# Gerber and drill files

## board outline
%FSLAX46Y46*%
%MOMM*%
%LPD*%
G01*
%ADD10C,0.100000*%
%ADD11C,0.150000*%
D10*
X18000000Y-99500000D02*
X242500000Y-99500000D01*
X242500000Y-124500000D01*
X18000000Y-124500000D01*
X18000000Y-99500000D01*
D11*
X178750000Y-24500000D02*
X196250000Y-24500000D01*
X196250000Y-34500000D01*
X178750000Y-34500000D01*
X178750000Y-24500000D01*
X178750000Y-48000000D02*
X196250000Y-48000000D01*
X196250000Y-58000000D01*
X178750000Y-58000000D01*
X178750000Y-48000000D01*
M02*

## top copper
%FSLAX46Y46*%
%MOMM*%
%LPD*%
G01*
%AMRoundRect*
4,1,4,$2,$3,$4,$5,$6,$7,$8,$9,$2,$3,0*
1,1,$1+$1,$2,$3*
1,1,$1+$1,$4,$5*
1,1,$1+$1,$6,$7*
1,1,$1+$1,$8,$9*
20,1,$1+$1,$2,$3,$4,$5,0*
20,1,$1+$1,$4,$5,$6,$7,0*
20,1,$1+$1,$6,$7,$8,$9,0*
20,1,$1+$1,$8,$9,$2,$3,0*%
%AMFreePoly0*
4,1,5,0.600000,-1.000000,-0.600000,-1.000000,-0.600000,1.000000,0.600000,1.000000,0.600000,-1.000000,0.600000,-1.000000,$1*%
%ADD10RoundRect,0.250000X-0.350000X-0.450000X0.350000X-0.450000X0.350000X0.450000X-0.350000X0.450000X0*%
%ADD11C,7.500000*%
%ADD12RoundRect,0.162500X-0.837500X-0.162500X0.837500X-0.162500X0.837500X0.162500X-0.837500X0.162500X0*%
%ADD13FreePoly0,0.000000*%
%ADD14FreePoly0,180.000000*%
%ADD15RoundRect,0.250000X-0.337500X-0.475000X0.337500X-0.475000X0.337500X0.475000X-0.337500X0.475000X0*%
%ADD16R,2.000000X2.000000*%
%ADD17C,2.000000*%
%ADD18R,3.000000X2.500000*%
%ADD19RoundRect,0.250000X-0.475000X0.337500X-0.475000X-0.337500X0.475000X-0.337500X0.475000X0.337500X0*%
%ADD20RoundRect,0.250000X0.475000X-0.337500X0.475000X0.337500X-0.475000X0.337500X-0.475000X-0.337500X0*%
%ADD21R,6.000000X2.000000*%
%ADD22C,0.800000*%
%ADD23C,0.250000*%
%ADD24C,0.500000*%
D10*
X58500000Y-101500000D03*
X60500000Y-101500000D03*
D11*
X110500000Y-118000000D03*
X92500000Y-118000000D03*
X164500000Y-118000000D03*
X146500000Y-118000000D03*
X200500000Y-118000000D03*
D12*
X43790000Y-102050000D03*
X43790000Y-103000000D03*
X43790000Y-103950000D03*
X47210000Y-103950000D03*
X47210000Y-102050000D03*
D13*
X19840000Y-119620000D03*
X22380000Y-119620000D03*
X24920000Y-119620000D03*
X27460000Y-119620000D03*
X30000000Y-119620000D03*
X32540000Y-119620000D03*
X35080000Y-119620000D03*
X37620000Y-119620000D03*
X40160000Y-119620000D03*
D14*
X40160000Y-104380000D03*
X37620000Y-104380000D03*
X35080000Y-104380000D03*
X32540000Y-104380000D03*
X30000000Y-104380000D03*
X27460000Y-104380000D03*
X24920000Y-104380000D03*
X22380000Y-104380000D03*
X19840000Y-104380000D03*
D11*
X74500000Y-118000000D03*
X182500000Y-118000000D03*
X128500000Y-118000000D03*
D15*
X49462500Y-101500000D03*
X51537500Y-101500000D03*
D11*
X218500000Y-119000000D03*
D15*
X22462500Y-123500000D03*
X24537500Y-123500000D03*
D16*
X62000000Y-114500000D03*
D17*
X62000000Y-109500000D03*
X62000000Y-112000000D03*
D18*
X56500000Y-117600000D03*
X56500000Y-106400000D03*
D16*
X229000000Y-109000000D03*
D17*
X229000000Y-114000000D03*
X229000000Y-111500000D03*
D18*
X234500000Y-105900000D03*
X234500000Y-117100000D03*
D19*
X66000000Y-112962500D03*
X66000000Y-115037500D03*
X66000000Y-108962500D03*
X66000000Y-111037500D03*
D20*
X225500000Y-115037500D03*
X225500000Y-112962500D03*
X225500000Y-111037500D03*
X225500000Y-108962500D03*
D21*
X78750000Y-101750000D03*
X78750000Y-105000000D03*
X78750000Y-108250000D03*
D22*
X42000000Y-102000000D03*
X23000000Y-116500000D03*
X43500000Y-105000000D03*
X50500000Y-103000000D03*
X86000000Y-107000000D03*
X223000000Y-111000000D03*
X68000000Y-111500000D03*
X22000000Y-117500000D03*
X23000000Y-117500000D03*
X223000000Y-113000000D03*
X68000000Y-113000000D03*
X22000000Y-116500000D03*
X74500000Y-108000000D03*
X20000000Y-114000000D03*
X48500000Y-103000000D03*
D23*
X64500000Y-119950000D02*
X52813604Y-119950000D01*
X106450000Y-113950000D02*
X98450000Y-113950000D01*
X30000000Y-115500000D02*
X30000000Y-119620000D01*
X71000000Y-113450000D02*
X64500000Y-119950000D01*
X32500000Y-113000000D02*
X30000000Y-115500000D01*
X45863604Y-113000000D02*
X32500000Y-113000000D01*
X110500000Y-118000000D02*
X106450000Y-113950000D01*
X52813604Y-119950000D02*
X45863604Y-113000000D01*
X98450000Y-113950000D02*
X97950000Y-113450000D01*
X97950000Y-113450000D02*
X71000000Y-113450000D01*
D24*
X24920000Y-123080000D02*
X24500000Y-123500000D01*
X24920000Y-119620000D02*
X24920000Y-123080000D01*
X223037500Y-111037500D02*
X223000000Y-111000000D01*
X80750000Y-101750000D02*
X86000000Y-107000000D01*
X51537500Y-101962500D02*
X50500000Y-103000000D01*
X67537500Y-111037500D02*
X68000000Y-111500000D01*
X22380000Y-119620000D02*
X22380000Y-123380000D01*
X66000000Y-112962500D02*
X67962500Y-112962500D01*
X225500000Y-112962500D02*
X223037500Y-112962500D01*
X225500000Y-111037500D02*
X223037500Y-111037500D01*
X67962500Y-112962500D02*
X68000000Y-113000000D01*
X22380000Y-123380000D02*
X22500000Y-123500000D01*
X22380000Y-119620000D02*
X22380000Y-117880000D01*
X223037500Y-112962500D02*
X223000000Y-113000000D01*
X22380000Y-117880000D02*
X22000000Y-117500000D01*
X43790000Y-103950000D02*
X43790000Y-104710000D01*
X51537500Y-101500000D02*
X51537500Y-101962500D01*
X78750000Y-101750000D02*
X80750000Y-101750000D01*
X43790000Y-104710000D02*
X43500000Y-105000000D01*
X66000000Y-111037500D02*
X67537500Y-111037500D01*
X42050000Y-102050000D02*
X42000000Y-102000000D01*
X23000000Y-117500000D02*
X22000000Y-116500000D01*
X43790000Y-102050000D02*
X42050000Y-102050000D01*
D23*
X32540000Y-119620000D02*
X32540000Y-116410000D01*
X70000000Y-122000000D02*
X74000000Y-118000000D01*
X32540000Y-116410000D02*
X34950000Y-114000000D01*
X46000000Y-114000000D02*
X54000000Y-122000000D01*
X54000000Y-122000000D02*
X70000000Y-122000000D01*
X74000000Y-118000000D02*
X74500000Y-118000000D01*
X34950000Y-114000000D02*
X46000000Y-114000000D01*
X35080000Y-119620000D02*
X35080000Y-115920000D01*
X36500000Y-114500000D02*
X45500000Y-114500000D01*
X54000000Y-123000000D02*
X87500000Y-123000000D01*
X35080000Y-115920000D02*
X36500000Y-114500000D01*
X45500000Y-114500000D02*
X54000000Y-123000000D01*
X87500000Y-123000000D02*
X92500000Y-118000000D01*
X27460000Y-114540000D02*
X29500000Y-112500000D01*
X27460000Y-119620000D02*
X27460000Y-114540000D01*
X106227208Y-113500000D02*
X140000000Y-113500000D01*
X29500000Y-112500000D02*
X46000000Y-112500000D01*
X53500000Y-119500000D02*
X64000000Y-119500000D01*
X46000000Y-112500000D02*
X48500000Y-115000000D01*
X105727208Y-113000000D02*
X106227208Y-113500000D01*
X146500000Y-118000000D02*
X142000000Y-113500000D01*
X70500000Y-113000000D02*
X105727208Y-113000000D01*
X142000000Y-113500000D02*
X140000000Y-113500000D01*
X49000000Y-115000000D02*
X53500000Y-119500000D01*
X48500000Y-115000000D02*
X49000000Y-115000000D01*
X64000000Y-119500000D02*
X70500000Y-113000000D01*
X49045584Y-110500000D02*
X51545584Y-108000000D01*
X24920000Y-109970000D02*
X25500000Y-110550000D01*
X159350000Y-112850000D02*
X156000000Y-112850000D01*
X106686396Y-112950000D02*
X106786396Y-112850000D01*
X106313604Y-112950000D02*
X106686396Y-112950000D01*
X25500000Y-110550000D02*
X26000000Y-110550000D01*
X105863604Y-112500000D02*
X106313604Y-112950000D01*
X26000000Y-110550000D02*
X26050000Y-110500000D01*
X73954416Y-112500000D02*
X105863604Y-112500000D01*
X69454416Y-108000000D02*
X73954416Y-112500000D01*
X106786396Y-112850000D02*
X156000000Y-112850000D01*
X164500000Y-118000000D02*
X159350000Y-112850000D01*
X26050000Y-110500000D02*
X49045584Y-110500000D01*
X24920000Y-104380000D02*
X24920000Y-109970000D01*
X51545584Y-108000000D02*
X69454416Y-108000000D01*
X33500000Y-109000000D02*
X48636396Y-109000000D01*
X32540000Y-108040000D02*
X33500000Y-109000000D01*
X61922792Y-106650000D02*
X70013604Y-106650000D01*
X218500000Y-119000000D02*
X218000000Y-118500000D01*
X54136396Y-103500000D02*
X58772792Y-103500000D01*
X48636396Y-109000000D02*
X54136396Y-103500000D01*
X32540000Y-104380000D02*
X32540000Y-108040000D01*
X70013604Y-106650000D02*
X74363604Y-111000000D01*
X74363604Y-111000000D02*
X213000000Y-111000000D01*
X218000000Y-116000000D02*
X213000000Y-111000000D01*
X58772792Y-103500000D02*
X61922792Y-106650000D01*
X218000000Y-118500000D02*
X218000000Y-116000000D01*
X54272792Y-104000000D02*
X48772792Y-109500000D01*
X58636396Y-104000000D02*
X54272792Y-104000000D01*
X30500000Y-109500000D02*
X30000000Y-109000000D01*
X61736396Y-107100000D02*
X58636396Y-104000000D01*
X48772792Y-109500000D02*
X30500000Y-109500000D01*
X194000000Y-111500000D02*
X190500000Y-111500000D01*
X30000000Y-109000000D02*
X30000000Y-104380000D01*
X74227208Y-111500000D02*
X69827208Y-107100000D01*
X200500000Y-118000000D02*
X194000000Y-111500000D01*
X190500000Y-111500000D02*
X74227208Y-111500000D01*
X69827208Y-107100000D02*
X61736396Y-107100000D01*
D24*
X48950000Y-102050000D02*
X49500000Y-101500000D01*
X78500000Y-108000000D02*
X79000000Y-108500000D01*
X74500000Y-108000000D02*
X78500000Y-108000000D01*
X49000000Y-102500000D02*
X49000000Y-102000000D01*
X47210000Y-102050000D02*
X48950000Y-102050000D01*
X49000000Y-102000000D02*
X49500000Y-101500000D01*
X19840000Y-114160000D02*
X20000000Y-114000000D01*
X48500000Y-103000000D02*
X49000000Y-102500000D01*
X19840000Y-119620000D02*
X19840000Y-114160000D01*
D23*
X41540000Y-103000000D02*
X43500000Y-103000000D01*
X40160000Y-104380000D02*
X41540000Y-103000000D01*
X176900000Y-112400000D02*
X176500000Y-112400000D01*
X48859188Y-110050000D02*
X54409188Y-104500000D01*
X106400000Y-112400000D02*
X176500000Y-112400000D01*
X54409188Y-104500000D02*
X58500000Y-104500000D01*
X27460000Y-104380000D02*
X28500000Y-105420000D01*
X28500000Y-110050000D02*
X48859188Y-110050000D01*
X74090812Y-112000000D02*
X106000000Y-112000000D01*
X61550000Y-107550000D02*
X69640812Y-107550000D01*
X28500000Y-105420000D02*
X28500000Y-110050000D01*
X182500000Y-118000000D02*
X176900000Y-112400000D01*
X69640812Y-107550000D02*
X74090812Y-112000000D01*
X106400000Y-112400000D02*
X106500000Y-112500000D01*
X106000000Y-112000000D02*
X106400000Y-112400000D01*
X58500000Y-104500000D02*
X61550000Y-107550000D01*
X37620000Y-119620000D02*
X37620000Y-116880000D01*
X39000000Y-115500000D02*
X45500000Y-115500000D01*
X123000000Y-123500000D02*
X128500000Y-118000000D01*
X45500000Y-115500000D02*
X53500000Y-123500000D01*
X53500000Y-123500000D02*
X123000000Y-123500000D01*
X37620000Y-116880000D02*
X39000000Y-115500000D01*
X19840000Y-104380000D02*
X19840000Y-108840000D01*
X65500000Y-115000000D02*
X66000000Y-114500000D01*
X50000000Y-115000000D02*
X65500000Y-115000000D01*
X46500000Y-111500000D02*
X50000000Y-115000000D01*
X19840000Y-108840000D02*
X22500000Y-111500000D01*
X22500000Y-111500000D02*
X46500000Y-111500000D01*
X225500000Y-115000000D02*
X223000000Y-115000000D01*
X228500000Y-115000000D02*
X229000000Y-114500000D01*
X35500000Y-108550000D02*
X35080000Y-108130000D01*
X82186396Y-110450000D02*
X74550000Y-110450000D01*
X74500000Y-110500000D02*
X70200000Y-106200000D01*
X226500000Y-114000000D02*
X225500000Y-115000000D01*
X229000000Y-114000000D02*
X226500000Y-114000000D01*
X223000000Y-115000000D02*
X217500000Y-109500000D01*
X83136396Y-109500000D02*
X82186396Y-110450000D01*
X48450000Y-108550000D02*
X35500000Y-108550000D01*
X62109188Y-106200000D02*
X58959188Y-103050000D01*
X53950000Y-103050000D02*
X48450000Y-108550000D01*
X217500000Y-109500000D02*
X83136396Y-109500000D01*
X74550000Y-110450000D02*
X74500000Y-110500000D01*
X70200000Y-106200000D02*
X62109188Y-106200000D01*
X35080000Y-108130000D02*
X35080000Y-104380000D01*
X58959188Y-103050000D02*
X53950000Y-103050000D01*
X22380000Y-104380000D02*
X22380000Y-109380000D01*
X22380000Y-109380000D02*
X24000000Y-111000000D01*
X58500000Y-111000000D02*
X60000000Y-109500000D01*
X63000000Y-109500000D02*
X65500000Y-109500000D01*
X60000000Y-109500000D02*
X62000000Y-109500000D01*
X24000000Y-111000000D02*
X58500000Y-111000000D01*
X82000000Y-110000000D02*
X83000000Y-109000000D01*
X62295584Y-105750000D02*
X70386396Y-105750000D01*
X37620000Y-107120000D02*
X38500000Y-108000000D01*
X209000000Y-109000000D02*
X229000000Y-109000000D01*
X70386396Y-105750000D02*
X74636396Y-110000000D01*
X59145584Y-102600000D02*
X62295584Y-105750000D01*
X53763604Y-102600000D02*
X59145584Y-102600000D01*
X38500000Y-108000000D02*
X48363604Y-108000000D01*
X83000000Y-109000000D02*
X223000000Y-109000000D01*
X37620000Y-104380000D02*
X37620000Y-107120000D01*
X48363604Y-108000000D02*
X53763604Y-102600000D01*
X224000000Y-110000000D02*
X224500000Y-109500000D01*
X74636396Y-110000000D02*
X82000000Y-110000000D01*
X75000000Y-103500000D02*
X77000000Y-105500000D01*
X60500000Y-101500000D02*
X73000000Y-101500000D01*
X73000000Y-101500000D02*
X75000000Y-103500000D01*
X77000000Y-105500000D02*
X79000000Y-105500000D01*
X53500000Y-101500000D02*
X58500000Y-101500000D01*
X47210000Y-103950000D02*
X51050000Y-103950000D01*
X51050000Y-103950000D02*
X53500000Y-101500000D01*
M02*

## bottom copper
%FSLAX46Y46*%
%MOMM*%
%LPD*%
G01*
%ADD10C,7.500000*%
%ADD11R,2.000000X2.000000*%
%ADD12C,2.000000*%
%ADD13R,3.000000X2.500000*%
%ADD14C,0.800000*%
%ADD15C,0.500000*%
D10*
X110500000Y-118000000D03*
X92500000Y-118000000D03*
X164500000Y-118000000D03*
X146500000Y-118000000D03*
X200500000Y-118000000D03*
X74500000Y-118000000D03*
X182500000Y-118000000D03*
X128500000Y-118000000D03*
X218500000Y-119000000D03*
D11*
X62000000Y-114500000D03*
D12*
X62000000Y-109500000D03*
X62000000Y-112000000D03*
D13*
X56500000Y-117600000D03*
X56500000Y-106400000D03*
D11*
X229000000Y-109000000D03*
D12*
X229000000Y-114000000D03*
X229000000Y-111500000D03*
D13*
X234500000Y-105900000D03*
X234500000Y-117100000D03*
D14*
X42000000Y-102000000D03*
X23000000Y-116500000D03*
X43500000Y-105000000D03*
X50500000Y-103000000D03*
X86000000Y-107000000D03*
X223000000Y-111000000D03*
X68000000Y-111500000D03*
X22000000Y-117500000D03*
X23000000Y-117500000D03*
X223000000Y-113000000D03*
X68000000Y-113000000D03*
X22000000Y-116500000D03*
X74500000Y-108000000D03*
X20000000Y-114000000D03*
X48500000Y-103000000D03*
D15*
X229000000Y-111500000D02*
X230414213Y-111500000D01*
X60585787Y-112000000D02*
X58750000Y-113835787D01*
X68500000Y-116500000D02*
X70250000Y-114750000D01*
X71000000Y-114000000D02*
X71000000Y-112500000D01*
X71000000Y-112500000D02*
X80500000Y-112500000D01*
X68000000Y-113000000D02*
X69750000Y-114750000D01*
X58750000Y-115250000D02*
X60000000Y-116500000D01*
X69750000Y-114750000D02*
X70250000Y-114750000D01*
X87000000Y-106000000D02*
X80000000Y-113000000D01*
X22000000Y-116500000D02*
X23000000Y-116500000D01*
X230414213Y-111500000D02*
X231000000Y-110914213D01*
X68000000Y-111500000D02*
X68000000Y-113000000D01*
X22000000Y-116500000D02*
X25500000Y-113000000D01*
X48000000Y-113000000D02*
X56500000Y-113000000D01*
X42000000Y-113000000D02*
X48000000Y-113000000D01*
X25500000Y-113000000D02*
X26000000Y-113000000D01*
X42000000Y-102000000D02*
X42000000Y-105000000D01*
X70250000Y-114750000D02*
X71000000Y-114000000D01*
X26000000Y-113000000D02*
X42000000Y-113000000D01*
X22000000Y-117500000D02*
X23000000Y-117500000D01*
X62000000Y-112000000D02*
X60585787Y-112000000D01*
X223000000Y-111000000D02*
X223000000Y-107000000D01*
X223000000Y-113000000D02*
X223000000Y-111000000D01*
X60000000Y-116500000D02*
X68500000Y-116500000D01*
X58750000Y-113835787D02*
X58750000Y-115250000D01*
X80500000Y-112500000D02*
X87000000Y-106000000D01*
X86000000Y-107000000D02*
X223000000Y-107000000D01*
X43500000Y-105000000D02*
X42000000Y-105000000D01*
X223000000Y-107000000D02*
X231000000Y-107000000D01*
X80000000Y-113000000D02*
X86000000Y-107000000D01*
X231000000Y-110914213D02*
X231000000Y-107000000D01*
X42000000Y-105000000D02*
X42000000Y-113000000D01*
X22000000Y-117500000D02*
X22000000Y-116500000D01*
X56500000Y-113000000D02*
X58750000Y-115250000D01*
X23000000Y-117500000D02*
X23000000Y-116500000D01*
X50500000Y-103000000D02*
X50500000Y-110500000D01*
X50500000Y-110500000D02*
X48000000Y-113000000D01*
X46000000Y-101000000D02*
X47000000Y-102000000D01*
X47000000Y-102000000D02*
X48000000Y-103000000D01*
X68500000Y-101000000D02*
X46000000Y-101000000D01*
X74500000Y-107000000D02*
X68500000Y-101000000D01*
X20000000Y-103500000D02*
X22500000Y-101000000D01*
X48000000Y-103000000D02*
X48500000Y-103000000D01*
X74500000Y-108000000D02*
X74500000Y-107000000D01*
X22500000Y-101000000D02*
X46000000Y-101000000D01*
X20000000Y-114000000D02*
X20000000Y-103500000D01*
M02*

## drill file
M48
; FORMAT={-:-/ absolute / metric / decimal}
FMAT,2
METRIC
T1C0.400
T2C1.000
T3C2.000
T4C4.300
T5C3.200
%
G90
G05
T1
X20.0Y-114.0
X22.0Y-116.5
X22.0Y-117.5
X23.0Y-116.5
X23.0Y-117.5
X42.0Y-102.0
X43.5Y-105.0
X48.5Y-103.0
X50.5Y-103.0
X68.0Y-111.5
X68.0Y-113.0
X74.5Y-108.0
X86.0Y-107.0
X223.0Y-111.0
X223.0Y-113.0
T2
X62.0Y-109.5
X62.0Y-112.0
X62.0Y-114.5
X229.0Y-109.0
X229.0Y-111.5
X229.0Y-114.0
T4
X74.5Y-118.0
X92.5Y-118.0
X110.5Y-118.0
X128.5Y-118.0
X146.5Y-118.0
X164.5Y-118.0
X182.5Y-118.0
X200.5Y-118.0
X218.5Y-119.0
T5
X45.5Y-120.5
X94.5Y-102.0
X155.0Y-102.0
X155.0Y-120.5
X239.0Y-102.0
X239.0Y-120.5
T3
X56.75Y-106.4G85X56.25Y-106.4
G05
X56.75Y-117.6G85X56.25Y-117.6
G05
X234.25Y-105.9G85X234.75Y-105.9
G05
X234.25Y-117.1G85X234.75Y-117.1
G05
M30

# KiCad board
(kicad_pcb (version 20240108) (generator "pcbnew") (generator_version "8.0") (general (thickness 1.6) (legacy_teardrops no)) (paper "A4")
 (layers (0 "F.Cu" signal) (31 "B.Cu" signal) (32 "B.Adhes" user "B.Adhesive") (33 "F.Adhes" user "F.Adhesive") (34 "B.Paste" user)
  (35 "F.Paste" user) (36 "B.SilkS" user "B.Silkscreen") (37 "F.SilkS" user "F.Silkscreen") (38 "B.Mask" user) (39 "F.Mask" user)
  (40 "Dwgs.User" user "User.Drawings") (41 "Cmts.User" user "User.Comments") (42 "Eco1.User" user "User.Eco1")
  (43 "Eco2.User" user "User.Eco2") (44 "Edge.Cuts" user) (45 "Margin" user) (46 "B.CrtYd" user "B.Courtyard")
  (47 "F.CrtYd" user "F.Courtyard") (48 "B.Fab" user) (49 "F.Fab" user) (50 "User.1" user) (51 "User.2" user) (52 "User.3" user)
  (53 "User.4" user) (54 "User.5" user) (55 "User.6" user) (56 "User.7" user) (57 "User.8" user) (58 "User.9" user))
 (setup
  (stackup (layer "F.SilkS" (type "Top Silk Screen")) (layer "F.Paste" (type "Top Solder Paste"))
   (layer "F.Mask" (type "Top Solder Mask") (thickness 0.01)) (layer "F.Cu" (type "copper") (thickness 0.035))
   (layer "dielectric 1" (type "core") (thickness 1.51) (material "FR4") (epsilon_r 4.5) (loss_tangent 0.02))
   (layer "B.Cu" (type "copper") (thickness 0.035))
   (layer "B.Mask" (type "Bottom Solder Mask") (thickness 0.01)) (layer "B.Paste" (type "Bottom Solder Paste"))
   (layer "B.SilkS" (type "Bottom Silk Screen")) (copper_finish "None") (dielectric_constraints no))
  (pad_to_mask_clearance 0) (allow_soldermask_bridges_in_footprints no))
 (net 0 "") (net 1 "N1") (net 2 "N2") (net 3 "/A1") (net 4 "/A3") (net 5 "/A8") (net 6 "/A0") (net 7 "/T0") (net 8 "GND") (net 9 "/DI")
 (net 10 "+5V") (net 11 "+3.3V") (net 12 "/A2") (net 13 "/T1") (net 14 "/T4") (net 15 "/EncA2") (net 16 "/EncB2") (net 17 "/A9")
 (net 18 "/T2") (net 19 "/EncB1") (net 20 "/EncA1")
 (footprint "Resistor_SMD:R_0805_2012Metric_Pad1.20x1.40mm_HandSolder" (layer "F.Cu") (at 59.5 101.5)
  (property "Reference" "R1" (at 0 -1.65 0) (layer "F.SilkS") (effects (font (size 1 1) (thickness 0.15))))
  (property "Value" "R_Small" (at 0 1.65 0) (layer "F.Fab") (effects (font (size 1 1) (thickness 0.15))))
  (pad "1" smd roundrect (at -1 0) (size 1.2 1.4) (layers "F.Cu" "F.Paste" "F.Mask") (roundrect_rratio 0.208333) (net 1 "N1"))
  (pad "2" smd roundrect (at 1 0) (size 1.2 1.4) (layers "F.Cu" "F.Paste" "F.Mask") (roundrect_rratio 0.208333) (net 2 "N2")))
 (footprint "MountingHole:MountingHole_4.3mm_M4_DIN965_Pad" (layer "F.Cu") (at 110.5 118)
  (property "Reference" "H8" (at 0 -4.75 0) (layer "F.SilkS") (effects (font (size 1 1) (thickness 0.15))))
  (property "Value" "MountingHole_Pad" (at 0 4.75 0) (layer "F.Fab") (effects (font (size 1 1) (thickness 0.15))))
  (pad "1" thru_hole circle (at 0 0) (size 7.5 7.5) (drill 4.3) (layers "*.Cu" "*.Mask") (remove_unused_layers no) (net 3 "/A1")))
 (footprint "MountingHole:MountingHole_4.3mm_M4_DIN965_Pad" (layer "F.Cu") (at 92.5 118)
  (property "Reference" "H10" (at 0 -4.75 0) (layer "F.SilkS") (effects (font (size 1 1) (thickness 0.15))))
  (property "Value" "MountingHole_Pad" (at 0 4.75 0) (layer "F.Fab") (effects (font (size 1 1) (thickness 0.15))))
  (pad "1" thru_hole circle (at 0 0) (size 7.5 7.5) (drill 4.3) (layers "*.Cu" "*.Mask") (remove_unused_layers no) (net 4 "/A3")))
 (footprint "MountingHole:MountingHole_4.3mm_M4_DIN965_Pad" (layer "F.Cu") (at 164.5 118)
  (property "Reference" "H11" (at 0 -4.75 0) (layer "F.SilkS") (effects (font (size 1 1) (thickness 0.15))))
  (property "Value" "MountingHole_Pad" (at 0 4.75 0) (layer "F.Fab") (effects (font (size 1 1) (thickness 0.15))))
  (pad "1" thru_hole circle (at 0 0) (size 7.5 7.5) (drill 4.3) (layers "*.Cu" "*.Mask") (remove_unused_layers no) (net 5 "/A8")))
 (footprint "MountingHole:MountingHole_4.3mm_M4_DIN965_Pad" (layer "F.Cu") (at 146.5 118)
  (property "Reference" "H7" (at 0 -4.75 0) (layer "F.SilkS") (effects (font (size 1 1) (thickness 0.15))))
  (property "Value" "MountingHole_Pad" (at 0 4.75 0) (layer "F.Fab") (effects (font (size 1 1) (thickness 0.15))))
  (pad "1" thru_hole circle (at 0 0) (size 7.5 7.5) (drill 4.3) (layers "*.Cu" "*.Mask") (remove_unused_layers no) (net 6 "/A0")))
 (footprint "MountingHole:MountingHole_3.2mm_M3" (layer "F.Cu") (at 238.5 102 90)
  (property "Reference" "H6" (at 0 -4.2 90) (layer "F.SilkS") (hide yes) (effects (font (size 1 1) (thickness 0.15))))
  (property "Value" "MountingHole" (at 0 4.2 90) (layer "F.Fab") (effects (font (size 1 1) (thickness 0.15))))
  (pad "" np_thru_hole circle (at 0 0.5 90) (size 3.2 3.2) (drill 3.2) (layers "F&B.Cu" "*.Mask")))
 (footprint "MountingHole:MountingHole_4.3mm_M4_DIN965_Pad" (layer "F.Cu") (at 200.5 118)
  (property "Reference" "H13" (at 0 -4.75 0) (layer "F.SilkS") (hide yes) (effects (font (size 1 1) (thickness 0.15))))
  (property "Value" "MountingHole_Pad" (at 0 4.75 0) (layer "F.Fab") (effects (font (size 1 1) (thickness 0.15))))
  (pad "1" thru_hole circle (at 0 0) (size 7.5 7.5) (drill 4.3) (layers "*.Cu" "*.Mask") (remove_unused_layers no) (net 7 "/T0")))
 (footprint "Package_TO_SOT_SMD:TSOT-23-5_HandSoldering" (layer "F.Cu") (at 45.5 103)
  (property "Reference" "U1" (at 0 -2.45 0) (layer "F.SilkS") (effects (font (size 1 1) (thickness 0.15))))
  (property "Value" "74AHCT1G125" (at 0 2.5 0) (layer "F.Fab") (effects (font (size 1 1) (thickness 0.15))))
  (pad "1" smd roundrect (at -1.71 -0.95) (size 2 0.65) (layers "F.Cu" "F.Paste" "F.Mask") (roundrect_rratio 0.25) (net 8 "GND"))
  (pad "2" smd roundrect (at -1.71 0) (size 2 0.65) (layers "F.Cu" "F.Paste" "F.Mask") (roundrect_rratio 0.25) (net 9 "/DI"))
  (pad "3" smd roundrect (at -1.71 0.95) (size 2 0.65) (layers "F.Cu" "F.Paste" "F.Mask") (roundrect_rratio 0.25) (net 8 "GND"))
  (pad "4" smd roundrect (at 1.71 0.95) (size 2 0.65) (layers "F.Cu" "F.Paste" "F.Mask") (roundrect_rratio 0.25) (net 1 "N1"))
  (pad "5" smd roundrect (at 1.71 -0.95) (size 2 0.65) (layers "F.Cu" "F.Paste" "F.Mask") (roundrect_rratio 0.25) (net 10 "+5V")))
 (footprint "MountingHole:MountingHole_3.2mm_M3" (layer "F.Cu") (at 239 121)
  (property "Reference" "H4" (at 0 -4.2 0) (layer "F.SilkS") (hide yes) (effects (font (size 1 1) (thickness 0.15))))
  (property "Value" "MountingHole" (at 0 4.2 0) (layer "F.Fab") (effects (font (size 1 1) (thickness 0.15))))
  (pad "" np_thru_hole circle (at 0 -0.5) (size 3.2 3.2) (drill 3.2) (layers "F&B.Cu" "*.Mask")))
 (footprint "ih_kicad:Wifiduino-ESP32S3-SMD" (layer "F.Cu") (at 30 112 90)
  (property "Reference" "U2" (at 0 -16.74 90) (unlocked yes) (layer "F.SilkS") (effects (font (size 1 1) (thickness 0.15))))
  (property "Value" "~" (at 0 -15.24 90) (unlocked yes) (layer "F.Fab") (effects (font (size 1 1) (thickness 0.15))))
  (pad "1" smd custom (at -7.62 -10.16) (size 1.2 2) (layers "F.Cu" "F.Paste" "F.Mask") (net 10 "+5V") (thermal_bridge_angle 45)
   (options (clearance outline) (anchor rect)) (primitives))
  (pad "2" smd custom (at -7.62 -7.62) (size 1.2 2) (layers "F.Cu" "F.Paste" "F.Mask") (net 8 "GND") (thermal_bridge_angle 45)
   (options (clearance outline) (anchor rect)) (primitives))
  (pad "3" smd custom (at -7.62 -5.08) (size 1.2 2) (layers "F.Cu" "F.Paste" "F.Mask") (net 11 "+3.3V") (thermal_bridge_angle 45)
   (options (clearance outline) (anchor rect)) (primitives))
  (pad "4" smd custom (at -7.62 -2.54) (size 1.2 2) (layers "F.Cu" "F.Paste" "F.Mask") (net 6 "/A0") (thermal_bridge_angle 45)
   (options (clearance outline) (anchor rect)) (primitives))
  (pad "5" smd custom (at -7.62 0) (size 1.2 2) (layers "F.Cu" "F.Paste" "F.Mask") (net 3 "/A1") (thermal_bridge_angle 45)
   (options (clearance outline) (anchor rect)) (primitives))
  (pad "6" smd custom (at -7.62 2.54) (size 1.2 2) (layers "F.Cu" "F.Paste" "F.Mask") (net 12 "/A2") (thermal_bridge_angle 45)
   (options (clearance outline) (anchor rect)) (primitives))
  (pad "7" smd custom (at -7.62 5.08) (size 1.2 2) (layers "F.Cu" "F.Paste" "F.Mask") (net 4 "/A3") (thermal_bridge_angle 45)
   (options (clearance outline) (anchor rect)) (primitives))
  (pad "8" smd custom (at -7.62 7.62) (size 1.2 2) (layers "F.Cu" "F.Paste" "F.Mask") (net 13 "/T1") (thermal_bridge_angle 45)
   (options (clearance outline) (anchor rect)) (primitives))
  (pad "9" smd custom (at -7.62 10.16) (size 1.2 2) (layers "F.Cu" "F.Paste" "F.Mask") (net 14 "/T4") (thermal_bridge_angle 45)
   (options (clearance outline) (anchor rect)) (primitives))
  (pad "10" smd custom (at 7.62 10.16 180) (size 1.2 2) (layers "F.Cu" "F.Paste" "F.Mask") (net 9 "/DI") (thermal_bridge_angle 45)
   (options (clearance outline) (anchor rect)) (primitives))
  (pad "11" smd custom (at 7.62 7.62 180) (size 1.2 2) (layers "F.Cu" "F.Paste" "F.Mask") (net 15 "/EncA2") (thermal_bridge_angle 45)
   (options (clearance outline) (anchor rect)) (primitives))
  (pad "12" smd custom (at 7.62 5.08 180) (size 1.2 2) (layers "F.Cu" "F.Paste" "F.Mask") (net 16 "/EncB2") (thermal_bridge_angle 45)
   (options (clearance outline) (anchor rect)) (primitives))
  (pad "13" smd custom (at 7.62 2.54 180) (size 1.2 2) (layers "F.Cu" "F.Paste" "F.Mask") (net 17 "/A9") (thermal_bridge_angle 45)
   (options (clearance outline) (anchor rect)) (primitives))
  (pad "14" smd custom (at 7.62 0 180) (size 1.2 2) (layers "F.Cu" "F.Paste" "F.Mask") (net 7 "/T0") (thermal_bridge_angle 45)
   (options (clearance outline) (anchor rect)) (primitives))
  (pad "15" smd custom (at 7.62 -2.54 180) (size 1.2 2) (layers "F.Cu" "F.Paste" "F.Mask") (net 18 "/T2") (thermal_bridge_angle 45)
   (options (clearance outline) (anchor rect)) (primitives))
  (pad "16" smd custom (at 7.62 -5.08 180) (size 1.2 2) (layers "F.Cu" "F.Paste" "F.Mask") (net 5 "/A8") (thermal_bridge_angle 45)
   (options (clearance outline) (anchor rect)) (primitives))
  (pad "17" smd custom (at 7.62 -7.62 180) (size 1.2 2) (layers "F.Cu" "F.Paste" "F.Mask") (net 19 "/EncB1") (thermal_bridge_angle 45)
   (options (clearance outline) (anchor rect)) (primitives))
  (pad "18" smd custom (at 7.62 -10.16 180) (size 1.2 2) (layers "F.Cu" "F.Paste" "F.Mask") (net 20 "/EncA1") (thermal_bridge_angle 45)
   (options (clearance outline) (anchor rect)) (primitives)))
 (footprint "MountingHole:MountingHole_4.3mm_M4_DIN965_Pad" (layer "F.Cu") (at 74.5 118)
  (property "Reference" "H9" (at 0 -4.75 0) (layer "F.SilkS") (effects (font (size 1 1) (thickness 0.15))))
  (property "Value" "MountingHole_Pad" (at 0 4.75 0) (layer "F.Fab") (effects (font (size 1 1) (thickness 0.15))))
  (pad "1" thru_hole circle (at 0 0) (size 7.5 7.5) (drill 4.3) (layers "*.Cu" "*.Mask") (remove_unused_layers no) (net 12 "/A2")))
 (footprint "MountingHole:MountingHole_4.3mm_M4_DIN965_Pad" (layer "F.Cu") (at 182.5 118)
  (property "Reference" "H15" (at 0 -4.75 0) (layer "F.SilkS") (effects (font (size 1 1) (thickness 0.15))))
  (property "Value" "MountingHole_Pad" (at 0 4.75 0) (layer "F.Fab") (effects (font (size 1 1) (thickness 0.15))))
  (pad "1" thru_hole circle (at 0 0) (size 7.5 7.5) (drill 4.3) (layers "*.Cu" "*.Mask") (remove_unused_layers no) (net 18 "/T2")))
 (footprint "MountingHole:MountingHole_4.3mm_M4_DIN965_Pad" (layer "F.Cu") (at 128.5 118)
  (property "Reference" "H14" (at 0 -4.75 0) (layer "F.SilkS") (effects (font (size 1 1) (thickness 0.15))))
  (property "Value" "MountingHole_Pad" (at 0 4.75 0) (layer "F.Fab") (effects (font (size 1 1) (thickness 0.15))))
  (pad "1" thru_hole circle (at 0 0) (size 7.5 7.5) (drill 4.3) (layers "*.Cu" "*.Mask") (remove_unused_layers no) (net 13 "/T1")))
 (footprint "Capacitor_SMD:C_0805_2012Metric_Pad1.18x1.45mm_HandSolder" (layer "F.Cu") (at 50.5 101.5)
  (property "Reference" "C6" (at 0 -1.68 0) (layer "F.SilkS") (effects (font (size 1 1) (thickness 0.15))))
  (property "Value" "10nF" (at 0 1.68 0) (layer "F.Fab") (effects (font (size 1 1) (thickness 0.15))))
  (pad "1" smd roundrect (at -1.0375 0) (size 1.175 1.45) (layers "F.Cu" "F.Paste" "F.Mask") (roundrect_rratio 0.212766) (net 10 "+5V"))
  (pad "2" smd roundrect (at 1.0375 0) (size 1.175 1.45) (layers "F.Cu" "F.Paste" "F.Mask") (roundrect_rratio 0.212766) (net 8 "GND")))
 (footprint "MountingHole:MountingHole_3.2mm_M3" (layer "F.Cu") (at 155 119)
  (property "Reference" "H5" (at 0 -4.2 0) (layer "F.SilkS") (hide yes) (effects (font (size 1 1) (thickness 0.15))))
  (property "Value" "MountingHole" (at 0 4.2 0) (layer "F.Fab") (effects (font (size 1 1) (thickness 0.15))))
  (pad "" np_thru_hole circle (at 0 1.5) (size 3.2 3.2) (drill 3.2) (layers "F&B.Cu" "*.Mask")))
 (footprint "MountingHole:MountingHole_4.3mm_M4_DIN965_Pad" (layer "F.Cu") (at 218.5 119)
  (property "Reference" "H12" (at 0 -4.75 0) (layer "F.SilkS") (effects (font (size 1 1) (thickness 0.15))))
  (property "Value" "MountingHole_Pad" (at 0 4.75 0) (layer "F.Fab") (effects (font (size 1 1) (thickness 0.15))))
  (pad "1" thru_hole circle (at 0 0) (size 7.5 7.5) (drill 4.3) (layers "*.Cu" "*.Mask") (remove_unused_layers no) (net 17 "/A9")))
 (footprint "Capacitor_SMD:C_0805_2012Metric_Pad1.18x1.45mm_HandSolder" (layer "F.Cu") (at 23.5 123.5)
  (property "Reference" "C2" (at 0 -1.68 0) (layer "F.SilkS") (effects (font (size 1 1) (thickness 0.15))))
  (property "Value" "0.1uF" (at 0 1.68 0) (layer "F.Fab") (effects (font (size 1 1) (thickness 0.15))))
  (pad "1" smd roundrect (at -1.0375 0) (size 1.175 1.45) (layers "F.Cu" "F.Paste" "F.Mask") (roundrect_rratio 0.212766) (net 8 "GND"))
  (pad "2" smd roundrect (at 1.0375 0) (size 1.175 1.45) (layers "F.Cu" "F.Paste" "F.Mask") (roundrect_rratio 0.212766) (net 11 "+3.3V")))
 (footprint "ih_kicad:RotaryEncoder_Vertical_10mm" (layer "F.Cu") (at 56.5 112 180)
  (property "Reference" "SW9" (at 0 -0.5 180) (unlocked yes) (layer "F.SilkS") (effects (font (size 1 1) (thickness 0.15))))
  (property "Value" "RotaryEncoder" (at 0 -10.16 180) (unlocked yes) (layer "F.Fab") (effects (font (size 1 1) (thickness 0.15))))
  (pad "A" thru_hole rect (at -5.5 -2.5 180) (size 2 2) (drill 1) (layers "*.Cu" "*.Mask") (remove_unused_layers no) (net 20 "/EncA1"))
  (pad "B" thru_hole circle (at -5.5 2.5 180) (size 2 2) (drill 1) (layers "*.Cu" "*.Mask") (remove_unused_layers no) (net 19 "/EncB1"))
  (pad "C" thru_hole circle (at -5.5 0 180) (size 2 2) (drill 1) (layers "*.Cu" "*.Mask") (remove_unused_layers no) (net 8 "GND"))
  (pad "MP" thru_hole rect (at 0 -5.6 180) (size 3 2.5) (drill oval 2.5 2) (layers "*.Cu" "*.Mask") (remove_unused_layers no))
  (pad "MP" thru_hole rect (at 0 5.6 180) (size 3 2.5) (drill oval 2.5 2) (layers "*.Cu" "*.Mask") (remove_unused_layers no)))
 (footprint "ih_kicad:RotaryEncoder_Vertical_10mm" (layer "F.Cu") (at 234.5 111.5)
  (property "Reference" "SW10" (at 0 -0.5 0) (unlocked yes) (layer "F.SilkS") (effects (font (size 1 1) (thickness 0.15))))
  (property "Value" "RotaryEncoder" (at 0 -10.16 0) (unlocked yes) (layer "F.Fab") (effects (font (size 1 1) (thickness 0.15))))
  (pad "A" thru_hole rect (at -5.5 -2.5) (size 2 2) (drill 1) (layers "*.Cu" "*.Mask") (remove_unused_layers no) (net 15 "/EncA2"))
  (pad "B" thru_hole circle (at -5.5 2.5) (size 2 2) (drill 1) (layers "*.Cu" "*.Mask") (remove_unused_layers no) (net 16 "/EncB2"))
  (pad "C" thru_hole circle (at -5.5 0) (size 2 2) (drill 1) (layers "*.Cu" "*.Mask") (remove_unused_layers no) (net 8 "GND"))
  (pad "MP" thru_hole rect (at 0 -5.6) (size 3 2.5) (drill oval 2.5 2) (layers "*.Cu" "*.Mask") (remove_unused_layers no))
  (pad "MP" thru_hole rect (at 0 5.6) (size 3 2.5) (drill oval 2.5 2) (layers "*.Cu" "*.Mask") (remove_unused_layers no)))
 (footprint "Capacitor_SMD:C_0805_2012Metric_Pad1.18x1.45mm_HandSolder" (layer "F.Cu") (at 66 114 -90)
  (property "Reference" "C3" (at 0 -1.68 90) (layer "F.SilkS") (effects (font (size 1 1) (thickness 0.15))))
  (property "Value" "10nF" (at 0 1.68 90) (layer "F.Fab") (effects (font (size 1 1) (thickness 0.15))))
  (pad "1" smd roundrect (at -1.0375 0 270) (size 1.175 1.45) (layers "F.Cu" "F.Paste" "F.Mask") (roundrect_rratio 0.212766) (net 8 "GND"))
  (pad "2" smd roundrect (at 1.0375 0 270) (size 1.175 1.45) (layers "F.Cu" "F.Paste" "F.Mask") (roundrect_rratio 0.212766)
   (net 20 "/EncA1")))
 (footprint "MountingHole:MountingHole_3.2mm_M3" (layer "F.Cu") (at 45.5 120.5)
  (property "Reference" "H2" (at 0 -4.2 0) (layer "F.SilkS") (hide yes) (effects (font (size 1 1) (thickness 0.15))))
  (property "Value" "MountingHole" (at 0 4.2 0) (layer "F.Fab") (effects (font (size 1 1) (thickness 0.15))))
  (pad "" np_thru_hole circle (at 0 0) (size 3.2 3.2) (drill 3.2) (layers "F&B.Cu" "*.Mask")))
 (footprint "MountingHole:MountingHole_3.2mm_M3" (layer "F.Cu") (at 94 104 90)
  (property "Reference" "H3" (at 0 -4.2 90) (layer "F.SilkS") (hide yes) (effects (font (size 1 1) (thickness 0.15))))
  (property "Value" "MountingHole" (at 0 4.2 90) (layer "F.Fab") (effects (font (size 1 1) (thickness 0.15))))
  (pad "" np_thru_hole circle (at 2 0.5 90) (size 3.2 3.2) (drill 3.2) (layers "F&B.Cu" "*.Mask")))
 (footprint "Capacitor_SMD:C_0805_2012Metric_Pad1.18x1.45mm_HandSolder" (layer "F.Cu") (at 66 110 -90)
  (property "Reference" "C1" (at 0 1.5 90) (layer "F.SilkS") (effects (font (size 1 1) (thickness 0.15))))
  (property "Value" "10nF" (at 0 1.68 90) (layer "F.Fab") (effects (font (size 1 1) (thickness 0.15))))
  (pad "1" smd roundrect (at -1.0375 0 270) (size 1.175 1.45) (layers "F.Cu" "F.Paste" "F.Mask") (roundrect_rratio 0.212766)
   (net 19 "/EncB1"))
  (pad "2" smd roundrect (at 1.0375 0 270) (size 1.175 1.45) (layers "F.Cu" "F.Paste" "F.Mask") (roundrect_rratio 0.212766) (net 8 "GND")))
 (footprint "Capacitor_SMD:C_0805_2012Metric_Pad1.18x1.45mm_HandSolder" (layer "F.Cu") (at 225.5 114 90)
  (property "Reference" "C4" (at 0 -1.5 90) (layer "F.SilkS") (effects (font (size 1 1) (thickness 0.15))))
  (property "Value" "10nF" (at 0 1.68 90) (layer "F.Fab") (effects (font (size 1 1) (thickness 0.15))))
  (pad "1" smd roundrect (at -1.0375 0 90) (size 1.175 1.45) (layers "F.Cu" "F.Paste" "F.Mask") (roundrect_rratio 0.212766)
   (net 16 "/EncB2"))
  (pad "2" smd roundrect (at 1.0375 0 90) (size 1.175 1.45) (layers "F.Cu" "F.Paste" "F.Mask") (roundrect_rratio 0.212766) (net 8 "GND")))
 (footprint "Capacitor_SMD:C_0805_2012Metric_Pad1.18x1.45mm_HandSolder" (layer "F.Cu") (at 225.5 110 90)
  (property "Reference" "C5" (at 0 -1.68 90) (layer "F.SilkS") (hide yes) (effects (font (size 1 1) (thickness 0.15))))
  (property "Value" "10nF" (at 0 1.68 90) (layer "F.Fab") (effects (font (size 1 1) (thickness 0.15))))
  (pad "1" smd roundrect (at -1.0375 0 90) (size 1.175 1.45) (layers "F.Cu" "F.Paste" "F.Mask") (roundrect_rratio 0.212766) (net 8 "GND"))
  (pad "2" smd roundrect (at 1.0375 0 90) (size 1.175 1.45) (layers "F.Cu" "F.Paste" "F.Mask") (roundrect_rratio 0.212766) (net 15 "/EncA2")))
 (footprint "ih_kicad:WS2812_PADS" (layer "F.Cu") (at 78.25 105 -90)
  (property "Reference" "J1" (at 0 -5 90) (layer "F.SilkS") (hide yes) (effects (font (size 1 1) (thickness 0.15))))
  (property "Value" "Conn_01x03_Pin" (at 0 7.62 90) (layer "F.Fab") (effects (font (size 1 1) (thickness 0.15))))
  (pad "1" smd rect (at -3.25 -0.5 270) (size 2 6) (layers "F.Cu" "F.Paste" "F.Mask") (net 8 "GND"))
  (pad "2" smd rect (at 0 -0.5 270) (size 2 6) (layers "F.Cu" "F.Paste" "F.Mask") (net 2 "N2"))
  (pad "3" smd rect (at 3.25 -0.5 270) (size 2 6) (layers "F.Cu" "F.Paste" "F.Mask") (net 10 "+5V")))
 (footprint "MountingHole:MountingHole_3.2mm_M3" (layer "F.Cu") (at 150.5 104)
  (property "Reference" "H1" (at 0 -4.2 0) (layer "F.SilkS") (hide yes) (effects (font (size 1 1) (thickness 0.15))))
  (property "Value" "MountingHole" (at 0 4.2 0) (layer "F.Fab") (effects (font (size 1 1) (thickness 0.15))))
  (pad "" np_thru_hole circle (at 4.5 -2) (size 3.2 3.2) (drill 3.2) (layers "F&B.Cu" "*.Mask")))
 (gr_rect (start 18 99.5) (end 242.5 124.5) (stroke (width 0.1) (type default)) (fill none) (layer "Edge.Cuts"))
 (gr_rect (start 178.75 24.5) (end 196.25 34.5) (stroke (width 0.15) (type default)) (fill none) (layer "Edge.Cuts"))
 (gr_rect (start 178.75 48) (end 196.25 58) (stroke (width 0.15) (type default)) (fill none) (layer "Edge.Cuts"))
 (segment (start 64.5 119.95) (end 52.813604 119.95) (width 0.25) (layer "F.Cu") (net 3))
 (segment (start 106.45 113.95) (end 98.45 113.95) (width 0.25) (layer "F.Cu") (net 3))
 (segment (start 30 115.5) (end 30 119.62) (width 0.25) (layer "F.Cu") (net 3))
 (segment (start 71 113.45) (end 64.5 119.95) (width 0.25) (layer "F.Cu") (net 3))
 (segment (start 32.5 113) (end 30 115.5) (width 0.25) (layer "F.Cu") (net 3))
 (segment (start 45.863604 113) (end 32.5 113) (width 0.25) (layer "F.Cu") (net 3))
 (segment (start 110.5 118) (end 106.45 113.95) (width 0.25) (layer "F.Cu") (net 3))
 (segment (start 52.813604 119.95) (end 45.863604 113) (width 0.25) (layer "F.Cu") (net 3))
 (segment (start 98.45 113.95) (end 97.95 113.45) (width 0.25) (layer "F.Cu") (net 3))
 (segment (start 97.95 113.45) (end 71 113.45) (width 0.25) (layer "F.Cu") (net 3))
 (segment (start 24.92 123.08) (end 24.5 123.5) (width 0.5) (layer "F.Cu") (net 11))
 (segment (start 24.92 119.62) (end 24.92 123.08) (width 0.5) (layer "F.Cu") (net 11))
 (segment (start 223.0375 111.0375) (end 223 111) (width 0.5) (layer "F.Cu") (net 8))
 (segment (start 80.75 101.75) (end 86 107) (width 0.5) (layer "F.Cu") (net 8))
 (segment (start 51.5375 101.9625) (end 50.5 103) (width 0.5) (layer "F.Cu") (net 8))
 (segment (start 67.5375 111.0375) (end 68 111.5) (width 0.5) (layer "F.Cu") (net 8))
 (segment (start 22.38 119.62) (end 22.38 123.38) (width 0.5) (layer "F.Cu") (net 8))
 (segment (start 66 112.9625) (end 67.9625 112.9625) (width 0.5) (layer "F.Cu") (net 8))
 (segment (start 225.5 112.9625) (end 223.0375 112.9625) (width 0.5) (layer "F.Cu") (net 8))
 (segment (start 225.5 111.0375) (end 223.0375 111.0375) (width 0.5) (layer "F.Cu") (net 8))
 (segment (start 67.9625 112.9625) (end 68 113) (width 0.5) (layer "F.Cu") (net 8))
 (segment (start 22.38 123.38) (end 22.5 123.5) (width 0.5) (layer "F.Cu") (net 8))
 (segment (start 22.38 119.62) (end 22.38 117.88) (width 0.5) (layer "F.Cu") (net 8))
 (segment (start 223.0375 112.9625) (end 223 113) (width 0.5) (layer "F.Cu") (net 8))
 (segment (start 22.38 117.88) (end 22 117.5) (width 0.5) (layer "F.Cu") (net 8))
 (segment (start 43.79 103.95) (end 43.79 104.71) (width 0.5) (layer "F.Cu") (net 8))
 (segment (start 51.5375 101.5) (end 51.5375 101.9625) (width 0.5) (layer "F.Cu") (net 8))
 (segment (start 78.75 101.75) (end 80.75 101.75) (width 0.5) (layer "F.Cu") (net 8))
 (segment (start 43.79 104.71) (end 43.5 105) (width 0.5) (layer "F.Cu") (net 8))
 (segment (start 66 111.0375) (end 67.5375 111.0375) (width 0.5) (layer "F.Cu") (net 8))
 (segment (start 42.05 102.05) (end 42 102) (width 0.5) (layer "F.Cu") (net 8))
 (segment (start 23 117.5) (end 22 116.5) (width 0.5) (layer "F.Cu") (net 8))
 (segment (start 43.79 102.05) (end 42.05 102.05) (width 0.5) (layer "F.Cu") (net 8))
 (via (at 42 102) (size 0.8) (drill 0.4) (layers "F.Cu" "B.Cu") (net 8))
 (via (at 23 116.5) (size 0.8) (drill 0.4) (layers "F.Cu" "B.Cu") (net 8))
 (via (at 43.5 105) (size 0.8) (drill 0.4) (layers "F.Cu" "B.Cu") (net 8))
 (via (at 50.5 103) (size 0.8) (drill 0.4) (layers "F.Cu" "B.Cu") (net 8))
 (via (at 86 107) (size 0.8) (drill 0.4) (layers "F.Cu" "B.Cu") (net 8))
 (via (at 223 111) (size 0.8) (drill 0.4) (layers "F.Cu" "B.Cu") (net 8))
 (via (at 68 111.5) (size 0.8) (drill 0.4) (layers "F.Cu" "B.Cu") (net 8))
 (via (at 22 117.5) (size 0.8) (drill 0.4) (layers "F.Cu" "B.Cu") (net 8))
 (via (at 23 117.5) (size 0.8) (drill 0.4) (layers "F.Cu" "B.Cu") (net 8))
 (via (at 223 113) (size 0.8) (drill 0.4) (layers "F.Cu" "B.Cu") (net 8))
 (via (at 68 113) (size 0.8) (drill 0.4) (layers "F.Cu" "B.Cu") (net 8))
 (via (at 22 116.5) (size 0.8) (drill 0.4) (layers "F.Cu" "B.Cu") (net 8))
 (segment (start 229 111.5) (end 230.414213 111.5) (width 0.5) (layer "B.Cu") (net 8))
 (segment (start 60.585787 112) (end 58.75 113.835787) (width 0.5) (layer "B.Cu") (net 8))
 (segment (start 68.5 116.5) (end 70.25 114.75) (width 0.5) (layer "B.Cu") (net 8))
 (segment (start 71 114) (end 71 112.5) (width 0.5) (layer "B.Cu") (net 8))
 (segment (start 71 112.5) (end 80.5 112.5) (width 0.5) (layer "B.Cu") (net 8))
 (segment (start 68 113) (end 69.75 114.75) (width 0.5) (layer "B.Cu") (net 8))
 (segment (start 58.75 115.25) (end 60 116.5) (width 0.5) (layer "B.Cu") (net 8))
 (segment (start 69.75 114.75) (end 70.25 114.75) (width 0.5) (layer "B.Cu") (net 8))
 (segment (start 87 106) (end 80 113) (width 0.5) (layer "B.Cu") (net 8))
 (segment (start 22 116.5) (end 23 116.5) (width 0.5) (layer "B.Cu") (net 8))
 (segment (start 230.414213 111.5) (end 231 110.914213) (width 0.5) (layer "B.Cu") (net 8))
 (segment (start 68 111.5) (end 68 113) (width 0.5) (layer "B.Cu") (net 8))
 (segment (start 22 116.5) (end 25.5 113) (width 0.5) (layer "B.Cu") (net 8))
 (segment (start 48 113) (end 56.5 113) (width 0.5) (layer "B.Cu") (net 8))
 (segment (start 42 113) (end 48 113) (width 0.5) (layer "B.Cu") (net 8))
 (segment (start 25.5 113) (end 26 113) (width 0.5) (layer "B.Cu") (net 8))
 (segment (start 42 102) (end 42 105) (width 0.5) (layer "B.Cu") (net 8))
 (segment (start 70.25 114.75) (end 71 114) (width 0.5) (layer "B.Cu") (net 8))
 (segment (start 26 113) (end 42 113) (width 0.5) (layer "B.Cu") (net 8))
 (segment (start 22 117.5) (end 23 117.5) (width 0.5) (layer "B.Cu") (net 8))
 (segment (start 62 112) (end 60.585787 112) (width 0.5) (layer "B.Cu") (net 8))
 (segment (start 223 111) (end 223 107) (width 0.5) (layer "B.Cu") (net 8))
 (segment (start 223 113) (end 223 111) (width 0.5) (layer "B.Cu") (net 8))
 (segment (start 60 116.5) (end 68.5 116.5) (width 0.5) (layer "B.Cu") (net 8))
 (segment (start 58.75 113.835787) (end 58.75 115.25) (width 0.5) (layer "B.Cu") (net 8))
 (segment (start 80.5 112.5) (end 87 106) (width 0.5) (layer "B.Cu") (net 8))
 (segment (start 86 107) (end 223 107) (width 0.5) (layer "B.Cu") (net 8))
 (segment (start 43.5 105) (end 42 105) (width 0.5) (layer "B.Cu") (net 8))
 (segment (start 223 107) (end 231 107) (width 0.5) (layer "B.Cu") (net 8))
 (segment (start 80 113) (end 86 107) (width 0.5) (layer "B.Cu") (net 8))
 (segment (start 231 110.914213) (end 231 107) (width 0.5) (layer "B.Cu") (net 8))
 (segment (start 42 105) (end 42 113) (width 0.5) (layer "B.Cu") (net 8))
 (segment (start 22 117.5) (end 22 116.5) (width 0.5) (layer "B.Cu") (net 8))
 (segment (start 56.5 113) (end 58.75 115.25) (width 0.5) (layer "B.Cu") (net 8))
 (segment (start 23 117.5) (end 23 116.5) (width 0.5) (layer "B.Cu") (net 8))
 (segment (start 50.5 103) (end 50.5 110.5) (width 0.5) (layer "B.Cu") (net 8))
 (segment (start 50.5 110.5) (end 48 113) (width 0.5) (layer "B.Cu") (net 8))
 (segment (start 32.54 119.62) (end 32.54 116.41) (width 0.25) (layer "F.Cu") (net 12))
 (segment (start 70 122) (end 74 118) (width 0.25) (layer "F.Cu") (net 12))
 (segment (start 32.54 116.41) (end 34.95 114) (width 0.25) (layer "F.Cu") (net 12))
 (segment (start 46 114) (end 54 122) (width 0.25) (layer "F.Cu") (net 12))
 (segment (start 54 122) (end 70 122) (width 0.25) (layer "F.Cu") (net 12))
 (segment (start 74 118) (end 74.5 118) (width 0.25) (layer "F.Cu") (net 12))
 (segment (start 34.95 114) (end 46 114) (width 0.25) (layer "F.Cu") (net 12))
 (segment (start 35.08 119.62) (end 35.08 115.92) (width 0.25) (layer "F.Cu") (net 4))
 (segment (start 36.5 114.5) (end 45.5 114.5) (width 0.25) (layer "F.Cu") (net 4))
 (segment (start 54 123) (end 87.5 123) (width 0.25) (layer "F.Cu") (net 4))
 (segment (start 35.08 115.92) (end 36.5 114.5) (width 0.25) (layer "F.Cu") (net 4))
 (segment (start 45.5 114.5) (end 54 123) (width 0.25) (layer "F.Cu") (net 4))
 (segment (start 87.5 123) (end 92.5 118) (width 0.25) (layer "F.Cu") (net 4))
 (segment (start 27.46 114.54) (end 29.5 112.5) (width 0.25) (layer "F.Cu") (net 6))
 (segment (start 27.46 119.62) (end 27.46 114.54) (width 0.25) (layer "F.Cu") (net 6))
 (segment (start 106.227208 113.5) (end 140 113.5) (width 0.25) (layer "F.Cu") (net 6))
 (segment (start 29.5 112.5) (end 46 112.5) (width 0.25) (layer "F.Cu") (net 6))
 (segment (start 53.5 119.5) (end 64 119.5) (width 0.25) (layer "F.Cu") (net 6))
 (segment (start 46 112.5) (end 48.5 115) (width 0.25) (layer "F.Cu") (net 6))
 (segment (start 105.727208 113) (end 106.227208 113.5) (width 0.25) (layer "F.Cu") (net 6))
 (segment (start 146.5 118) (end 142 113.5) (width 0.25) (layer "F.Cu") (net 6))
 (segment (start 70.5 113) (end 105.727208 113) (width 0.25) (layer "F.Cu") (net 6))
 (segment (start 142 113.5) (end 140 113.5) (width 0.25) (layer "F.Cu") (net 6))
 (segment (start 49 115) (end 53.5 119.5) (width 0.25) (layer "F.Cu") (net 6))
 (segment (start 48.5 115) (end 49 115) (width 0.25) (layer "F.Cu") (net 6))
 (segment (start 64 119.5) (end 70.5 113) (width 0.25) (layer "F.Cu") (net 6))
 (segment (start 49.045584 110.5) (end 51.545584 108) (width 0.25) (layer "F.Cu") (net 5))
 (segment (start 24.92 109.97) (end 25.5 110.55) (width 0.25) (layer "F.Cu") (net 5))
 (segment (start 159.35 112.85) (end 156 112.85) (width 0.25) (layer "F.Cu") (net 5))
 (segment (start 106.686396 112.95) (end 106.786396 112.85) (width 0.25) (layer "F.Cu") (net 5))
 (segment (start 106.313604 112.95) (end 106.686396 112.95) (width 0.25) (layer "F.Cu") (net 5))
 (segment (start 25.5 110.55) (end 26 110.55) (width 0.25) (layer "F.Cu") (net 5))
 (segment (start 105.863604 112.5) (end 106.313604 112.95) (width 0.25) (layer "F.Cu") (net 5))
 (segment (start 26 110.55) (end 26.05 110.5) (width 0.25) (layer "F.Cu") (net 5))
 (segment (start 73.954416 112.5) (end 105.863604 112.5) (width 0.25) (layer "F.Cu") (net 5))
 (segment (start 69.454416 108) (end 73.954416 112.5) (width 0.25) (layer "F.Cu") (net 5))
 (segment (start 106.786396 112.85) (end 156 112.85) (width 0.25) (layer "F.Cu") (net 5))
 (segment (start 164.5 118) (end 159.35 112.85) (width 0.25) (layer "F.Cu") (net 5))
 (segment (start 26.05 110.5) (end 49.045584 110.5) (width 0.25) (layer "F.Cu") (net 5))
 (segment (start 24.92 104.38) (end 24.92 109.97) (width 0.25) (layer "F.Cu") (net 5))
 (segment (start 51.545584 108) (end 69.454416 108) (width 0.25) (layer "F.Cu") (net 5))
 (segment (start 33.5 109) (end 48.636396 109) (width 0.25) (layer "F.Cu") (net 17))
 (segment (start 32.54 108.04) (end 33.5 109) (width 0.25) (layer "F.Cu") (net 17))
 (segment (start 61.922792 106.65) (end 70.013604 106.65) (width 0.25) (layer "F.Cu") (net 17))
 (segment (start 218.5 119) (end 218 118.5) (width 0.25) (layer "F.Cu") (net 17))
 (segment (start 54.136396 103.5) (end 58.772792 103.5) (width 0.25) (layer "F.Cu") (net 17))
 (segment (start 48.636396 109) (end 54.136396 103.5) (width 0.25) (layer "F.Cu") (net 17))
 (segment (start 32.54 104.38) (end 32.54 108.04) (width 0.25) (layer "F.Cu") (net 17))
 (segment (start 70.013604 106.65) (end 74.363604 111) (width 0.25) (layer "F.Cu") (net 17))
 (segment (start 74.363604 111) (end 213 111) (width 0.25) (layer "F.Cu") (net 17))
 (segment (start 218 116) (end 213 111) (width 0.25) (layer "F.Cu") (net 17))
 (segment (start 58.772792 103.5) (end 61.922792 106.65) (width 0.25) (layer "F.Cu") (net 17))
 (segment (start 218 118.5) (end 218 116) (width 0.25) (layer "F.Cu") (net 17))
 (segment (start 54.272792 104) (end 48.772792 109.5) (width 0.25) (layer "F.Cu") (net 7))
 (segment (start 58.636396 104) (end 54.272792 104) (width 0.25) (layer "F.Cu") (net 7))
 (segment (start 30.5 109.5) (end 30 109) (width 0.25) (layer "F.Cu") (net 7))
 (segment (start 61.736396 107.1) (end 58.636396 104) (width 0.25) (layer "F.Cu") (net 7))
 (segment (start 48.772792 109.5) (end 30.5 109.5) (width 0.25) (layer "F.Cu") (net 7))
 (segment (start 194 111.5) (end 190.5 111.5) (width 0.25) (layer "F.Cu") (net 7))
 (segment (start 30 109) (end 30 104.38) (width 0.25) (layer "F.Cu") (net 7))
 (segment (start 74.227208 111.5) (end 69.827208 107.1) (width 0.25) (layer "F.Cu") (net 7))
 (segment (start 200.5 118) (end 194 111.5) (width 0.25) (layer "F.Cu") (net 7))
 (segment (start 190.5 111.5) (end 74.227208 111.5) (width 0.25) (layer "F.Cu") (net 7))
 (segment (start 69.827208 107.1) (end 61.736396 107.1) (width 0.25) (layer "F.Cu") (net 7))
 (segment (start 48.95 102.05) (end 49.5 101.5) (width 0.5) (layer "F.Cu") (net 10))
 (segment (start 78.5 108) (end 79 108.5) (width 0.5) (layer "F.Cu") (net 10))
 (segment (start 74.5 108) (end 78.5 108) (width 0.5) (layer "F.Cu") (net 10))
 (segment (start 49 102.5) (end 49 102) (width 0.5) (layer "F.Cu") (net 10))
 (segment (start 47.21 102.05) (end 48.95 102.05) (width 0.5) (layer "F.Cu") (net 10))
 (segment (start 49 102) (end 49.5 101.5) (width 0.5) (layer "F.Cu") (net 10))
 (segment (start 19.84 114.16) (end 20 114) (width 0.5) (layer "F.Cu") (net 10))
 (segment (start 48.5 103) (end 49 102.5) (width 0.5) (layer "F.Cu") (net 10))
 (segment (start 19.84 119.62) (end 19.84 114.16) (width 0.5) (layer "F.Cu") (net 10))
 (via (at 74.5 108) (size 0.8) (drill 0.4) (layers "F.Cu" "B.Cu") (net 10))
 (via (at 20 114) (size 0.8) (drill 0.4) (layers "F.Cu" "B.Cu") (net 10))
 (via (at 48.5 103) (size 0.8) (drill 0.4) (layers "F.Cu" "B.Cu") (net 10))
 (segment (start 46 101) (end 47 102) (width 0.5) (layer "B.Cu") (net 10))
 (segment (start 47 102) (end 48 103) (width 0.5) (layer "B.Cu") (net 10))
 (segment (start 68.5 101) (end 46 101) (width 0.5) (layer "B.Cu") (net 10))
 (segment (start 74.5 107) (end 68.5 101) (width 0.5) (layer "B.Cu") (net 10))
 (segment (start 20 103.5) (end 22.5 101) (width 0.5) (layer "B.Cu") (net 10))
 (segment (start 48 103) (end 48.5 103) (width 0.5) (layer "B.Cu") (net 10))
 (segment (start 74.5 108) (end 74.5 107) (width 0.5) (layer "B.Cu") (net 10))
 (segment (start 22.5 101) (end 46 101) (width 0.5) (layer "B.Cu") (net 10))
 (segment (start 20 114) (end 20 103.5) (width 0.5) (layer "B.Cu") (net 10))
 (segment (start 41.54 103) (end 43.5 103) (width 0.25) (layer "F.Cu") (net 9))
 (segment (start 40.16 104.38) (end 41.54 103) (width 0.25) (layer "F.Cu") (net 9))
 (segment (start 176.9 112.4) (end 176.5 112.4) (width 0.25) (layer "F.Cu") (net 18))
 (segment (start 48.859188 110.05) (end 54.409188 104.5) (width 0.25) (layer "F.Cu") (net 18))
 (segment (start 106.4 112.4) (end 176.5 112.4) (width 0.25) (layer "F.Cu") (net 18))
 (segment (start 54.409188 104.5) (end 58.5 104.5) (width 0.25) (layer "F.Cu") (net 18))
 (segment (start 27.46 104.38) (end 28.5 105.42) (width 0.25) (layer "F.Cu") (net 18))
 (segment (start 28.5 110.05) (end 48.859188 110.05) (width 0.25) (layer "F.Cu") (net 18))
 (segment (start 74.090812 112) (end 106 112) (width 0.25) (layer "F.Cu") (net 18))
 (segment (start 61.55 107.55) (end 69.640812 107.55) (width 0.25) (layer "F.Cu") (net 18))
 (segment (start 28.5 105.42) (end 28.5 110.05) (width 0.25) (layer "F.Cu") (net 18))
 (segment (start 182.5 118) (end 176.9 112.4) (width 0.25) (layer "F.Cu") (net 18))
 (segment (start 69.640812 107.55) (end 74.090812 112) (width 0.25) (layer "F.Cu") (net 18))
 (segment (start 106.4 112.4) (end 106.5 112.5) (width 0.25) (layer "F.Cu") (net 18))
 (segment (start 106 112) (end 106.4 112.4) (width 0.25) (layer "F.Cu") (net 18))
 (segment (start 58.5 104.5) (end 61.55 107.55) (width 0.25) (layer "F.Cu") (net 18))
 (segment (start 37.62 119.62) (end 37.62 116.88) (width 0.25) (layer "F.Cu") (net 13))
 (segment (start 39 115.5) (end 45.5 115.5) (width 0.25) (layer "F.Cu") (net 13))
 (segment (start 123 123.5) (end 128.5 118) (width 0.25) (layer "F.Cu") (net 13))
 (segment (start 45.5 115.5) (end 53.5 123.5) (width 0.25) (layer "F.Cu") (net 13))
 (segment (start 53.5 123.5) (end 123 123.5) (width 0.25) (layer "F.Cu") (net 13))
 (segment (start 37.62 116.88) (end 39 115.5) (width 0.25) (layer "F.Cu") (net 13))
 (segment (start 19.84 104.38) (end 19.84 108.84) (width 0.25) (layer "F.Cu") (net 20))
 (segment (start 65.5 115) (end 66 114.5) (width 0.25) (layer "F.Cu") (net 20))
 (segment (start 50 115) (end 65.5 115) (width 0.25) (layer "F.Cu") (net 20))
 (segment (start 46.5 111.5) (end 50 115) (width 0.25) (layer "F.Cu") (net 20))
 (segment (start 19.84 108.84) (end 22.5 111.5) (width 0.25) (layer "F.Cu") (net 20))
 (segment (start 22.5 111.5) (end 46.5 111.5) (width 0.25) (layer "F.Cu") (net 20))
 (segment (start 225.5 115) (end 223 115) (width 0.25) (layer "F.Cu") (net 16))
 (segment (start 228.5 115) (end 229 114.5) (width 0.25) (layer "F.Cu") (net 16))
 (segment (start 35.5 108.55) (end 35.08 108.13) (width 0.25) (layer "F.Cu") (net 16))
 (segment (start 82.186396 110.45) (end 74.55 110.45) (width 0.25) (layer "F.Cu") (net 16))
 (segment (start 74.5 110.5) (end 70.2 106.2) (width 0.25) (layer "F.Cu") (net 16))
 (segment (start 226.5 114) (end 225.5 115) (width 0.25) (layer "F.Cu") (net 16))
 (segment (start 229 114) (end 226.5 114) (width 0.25) (layer "F.Cu") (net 16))
 (segment (start 223 115) (end 217.5 109.5) (width 0.25) (layer "F.Cu") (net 16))
 (segment (start 83.136396 109.5) (end 82.186396 110.45) (width 0.25) (layer "F.Cu") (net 16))
 (segment (start 48.45 108.55) (end 35.5 108.55) (width 0.25) (layer "F.Cu") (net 16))
 (segment (start 62.109188 106.2) (end 58.959188 103.05) (width 0.25) (layer "F.Cu") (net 16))
 (segment (start 53.95 103.05) (end 48.45 108.55) (width 0.25) (layer "F.Cu") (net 16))
 (segment (start 217.5 109.5) (end 83.136396 109.5) (width 0.25) (layer "F.Cu") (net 16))
 (segment (start 74.55 110.45) (end 74.5 110.5) (width 0.25) (layer "F.Cu") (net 16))
 (segment (start 70.2 106.2) (end 62.109188 106.2) (width 0.25) (layer "F.Cu") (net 16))
 (segment (start 35.08 108.13) (end 35.08 104.38) (width 0.25) (layer "F.Cu") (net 16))
 (segment (start 58.959188 103.05) (end 53.95 103.05) (width 0.25) (layer "F.Cu") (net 16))
 (segment (start 22.38 104.38) (end 22.38 109.38) (width 0.25) (layer "F.Cu") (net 19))
 (segment (start 22.38 109.38) (end 24 111) (width 0.25) (layer "F.Cu") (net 19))
 (segment (start 58.5 111) (end 60 109.5) (width 0.25) (layer "F.Cu") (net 19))
 (segment (start 63 109.5) (end 65.5 109.5) (width 0.25) (layer "F.Cu") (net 19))
 (segment (start 60 109.5) (end 62 109.5) (width 0.25) (layer "F.Cu") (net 19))
 (segment (start 24 111) (end 58.5 111) (width 0.25) (layer "F.Cu") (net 19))
 (segment (start 82 110) (end 83 109) (width 0.25) (layer "F.Cu") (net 15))
 (segment (start 62.295584 105.75) (end 70.386396 105.75) (width 0.25) (layer "F.Cu") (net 15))
 (segment (start 37.62 107.12) (end 38.5 108) (width 0.25) (layer "F.Cu") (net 15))
 (segment (start 209 109) (end 229 109) (width 0.25) (layer "F.Cu") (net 15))
 (segment (start 70.386396 105.75) (end 74.636396 110) (width 0.25) (layer "F.Cu") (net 15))
 (segment (start 59.145584 102.6) (end 62.295584 105.75) (width 0.25) (layer "F.Cu") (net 15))
 (segment (start 53.763604 102.6) (end 59.145584 102.6) (width 0.25) (layer "F.Cu") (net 15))
 (segment (start 38.5 108) (end 48.363604 108) (width 0.25) (layer "F.Cu") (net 15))
 (segment (start 83 109) (end 223 109) (width 0.25) (layer "F.Cu") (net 15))
 (segment (start 37.62 104.38) (end 37.62 107.12) (width 0.25) (layer "F.Cu") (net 15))
 (segment (start 48.363604 108) (end 53.763604 102.6) (width 0.25) (layer "F.Cu") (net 15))
 (segment (start 224 110) (end 224.5 109.5) (width 0.25) (layer "F.Cu") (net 15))
 (segment (start 74.636396 110) (end 82 110) (width 0.25) (layer "F.Cu") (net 15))
 (segment (start 75 103.5) (end 77 105.5) (width 0.25) (layer "F.Cu") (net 2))
 (segment (start 60.5 101.5) (end 73 101.5) (width 0.25) (layer "F.Cu") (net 2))
 (segment (start 73 101.5) (end 75 103.5) (width 0.25) (layer "F.Cu") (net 2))
 (segment (start 77 105.5) (end 79 105.5) (width 0.25) (layer "F.Cu") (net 2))
 (segment (start 53.5 101.5) (end 58.5 101.5) (width 0.25) (layer "F.Cu") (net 1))
 (segment (start 47.21 103.95) (end 51.05 103.95) (width 0.25) (layer "F.Cu") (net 1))
 (segment (start 51.05 103.95) (end 53.5 101.5) (width 0.25) (layer "F.Cu") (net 1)))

